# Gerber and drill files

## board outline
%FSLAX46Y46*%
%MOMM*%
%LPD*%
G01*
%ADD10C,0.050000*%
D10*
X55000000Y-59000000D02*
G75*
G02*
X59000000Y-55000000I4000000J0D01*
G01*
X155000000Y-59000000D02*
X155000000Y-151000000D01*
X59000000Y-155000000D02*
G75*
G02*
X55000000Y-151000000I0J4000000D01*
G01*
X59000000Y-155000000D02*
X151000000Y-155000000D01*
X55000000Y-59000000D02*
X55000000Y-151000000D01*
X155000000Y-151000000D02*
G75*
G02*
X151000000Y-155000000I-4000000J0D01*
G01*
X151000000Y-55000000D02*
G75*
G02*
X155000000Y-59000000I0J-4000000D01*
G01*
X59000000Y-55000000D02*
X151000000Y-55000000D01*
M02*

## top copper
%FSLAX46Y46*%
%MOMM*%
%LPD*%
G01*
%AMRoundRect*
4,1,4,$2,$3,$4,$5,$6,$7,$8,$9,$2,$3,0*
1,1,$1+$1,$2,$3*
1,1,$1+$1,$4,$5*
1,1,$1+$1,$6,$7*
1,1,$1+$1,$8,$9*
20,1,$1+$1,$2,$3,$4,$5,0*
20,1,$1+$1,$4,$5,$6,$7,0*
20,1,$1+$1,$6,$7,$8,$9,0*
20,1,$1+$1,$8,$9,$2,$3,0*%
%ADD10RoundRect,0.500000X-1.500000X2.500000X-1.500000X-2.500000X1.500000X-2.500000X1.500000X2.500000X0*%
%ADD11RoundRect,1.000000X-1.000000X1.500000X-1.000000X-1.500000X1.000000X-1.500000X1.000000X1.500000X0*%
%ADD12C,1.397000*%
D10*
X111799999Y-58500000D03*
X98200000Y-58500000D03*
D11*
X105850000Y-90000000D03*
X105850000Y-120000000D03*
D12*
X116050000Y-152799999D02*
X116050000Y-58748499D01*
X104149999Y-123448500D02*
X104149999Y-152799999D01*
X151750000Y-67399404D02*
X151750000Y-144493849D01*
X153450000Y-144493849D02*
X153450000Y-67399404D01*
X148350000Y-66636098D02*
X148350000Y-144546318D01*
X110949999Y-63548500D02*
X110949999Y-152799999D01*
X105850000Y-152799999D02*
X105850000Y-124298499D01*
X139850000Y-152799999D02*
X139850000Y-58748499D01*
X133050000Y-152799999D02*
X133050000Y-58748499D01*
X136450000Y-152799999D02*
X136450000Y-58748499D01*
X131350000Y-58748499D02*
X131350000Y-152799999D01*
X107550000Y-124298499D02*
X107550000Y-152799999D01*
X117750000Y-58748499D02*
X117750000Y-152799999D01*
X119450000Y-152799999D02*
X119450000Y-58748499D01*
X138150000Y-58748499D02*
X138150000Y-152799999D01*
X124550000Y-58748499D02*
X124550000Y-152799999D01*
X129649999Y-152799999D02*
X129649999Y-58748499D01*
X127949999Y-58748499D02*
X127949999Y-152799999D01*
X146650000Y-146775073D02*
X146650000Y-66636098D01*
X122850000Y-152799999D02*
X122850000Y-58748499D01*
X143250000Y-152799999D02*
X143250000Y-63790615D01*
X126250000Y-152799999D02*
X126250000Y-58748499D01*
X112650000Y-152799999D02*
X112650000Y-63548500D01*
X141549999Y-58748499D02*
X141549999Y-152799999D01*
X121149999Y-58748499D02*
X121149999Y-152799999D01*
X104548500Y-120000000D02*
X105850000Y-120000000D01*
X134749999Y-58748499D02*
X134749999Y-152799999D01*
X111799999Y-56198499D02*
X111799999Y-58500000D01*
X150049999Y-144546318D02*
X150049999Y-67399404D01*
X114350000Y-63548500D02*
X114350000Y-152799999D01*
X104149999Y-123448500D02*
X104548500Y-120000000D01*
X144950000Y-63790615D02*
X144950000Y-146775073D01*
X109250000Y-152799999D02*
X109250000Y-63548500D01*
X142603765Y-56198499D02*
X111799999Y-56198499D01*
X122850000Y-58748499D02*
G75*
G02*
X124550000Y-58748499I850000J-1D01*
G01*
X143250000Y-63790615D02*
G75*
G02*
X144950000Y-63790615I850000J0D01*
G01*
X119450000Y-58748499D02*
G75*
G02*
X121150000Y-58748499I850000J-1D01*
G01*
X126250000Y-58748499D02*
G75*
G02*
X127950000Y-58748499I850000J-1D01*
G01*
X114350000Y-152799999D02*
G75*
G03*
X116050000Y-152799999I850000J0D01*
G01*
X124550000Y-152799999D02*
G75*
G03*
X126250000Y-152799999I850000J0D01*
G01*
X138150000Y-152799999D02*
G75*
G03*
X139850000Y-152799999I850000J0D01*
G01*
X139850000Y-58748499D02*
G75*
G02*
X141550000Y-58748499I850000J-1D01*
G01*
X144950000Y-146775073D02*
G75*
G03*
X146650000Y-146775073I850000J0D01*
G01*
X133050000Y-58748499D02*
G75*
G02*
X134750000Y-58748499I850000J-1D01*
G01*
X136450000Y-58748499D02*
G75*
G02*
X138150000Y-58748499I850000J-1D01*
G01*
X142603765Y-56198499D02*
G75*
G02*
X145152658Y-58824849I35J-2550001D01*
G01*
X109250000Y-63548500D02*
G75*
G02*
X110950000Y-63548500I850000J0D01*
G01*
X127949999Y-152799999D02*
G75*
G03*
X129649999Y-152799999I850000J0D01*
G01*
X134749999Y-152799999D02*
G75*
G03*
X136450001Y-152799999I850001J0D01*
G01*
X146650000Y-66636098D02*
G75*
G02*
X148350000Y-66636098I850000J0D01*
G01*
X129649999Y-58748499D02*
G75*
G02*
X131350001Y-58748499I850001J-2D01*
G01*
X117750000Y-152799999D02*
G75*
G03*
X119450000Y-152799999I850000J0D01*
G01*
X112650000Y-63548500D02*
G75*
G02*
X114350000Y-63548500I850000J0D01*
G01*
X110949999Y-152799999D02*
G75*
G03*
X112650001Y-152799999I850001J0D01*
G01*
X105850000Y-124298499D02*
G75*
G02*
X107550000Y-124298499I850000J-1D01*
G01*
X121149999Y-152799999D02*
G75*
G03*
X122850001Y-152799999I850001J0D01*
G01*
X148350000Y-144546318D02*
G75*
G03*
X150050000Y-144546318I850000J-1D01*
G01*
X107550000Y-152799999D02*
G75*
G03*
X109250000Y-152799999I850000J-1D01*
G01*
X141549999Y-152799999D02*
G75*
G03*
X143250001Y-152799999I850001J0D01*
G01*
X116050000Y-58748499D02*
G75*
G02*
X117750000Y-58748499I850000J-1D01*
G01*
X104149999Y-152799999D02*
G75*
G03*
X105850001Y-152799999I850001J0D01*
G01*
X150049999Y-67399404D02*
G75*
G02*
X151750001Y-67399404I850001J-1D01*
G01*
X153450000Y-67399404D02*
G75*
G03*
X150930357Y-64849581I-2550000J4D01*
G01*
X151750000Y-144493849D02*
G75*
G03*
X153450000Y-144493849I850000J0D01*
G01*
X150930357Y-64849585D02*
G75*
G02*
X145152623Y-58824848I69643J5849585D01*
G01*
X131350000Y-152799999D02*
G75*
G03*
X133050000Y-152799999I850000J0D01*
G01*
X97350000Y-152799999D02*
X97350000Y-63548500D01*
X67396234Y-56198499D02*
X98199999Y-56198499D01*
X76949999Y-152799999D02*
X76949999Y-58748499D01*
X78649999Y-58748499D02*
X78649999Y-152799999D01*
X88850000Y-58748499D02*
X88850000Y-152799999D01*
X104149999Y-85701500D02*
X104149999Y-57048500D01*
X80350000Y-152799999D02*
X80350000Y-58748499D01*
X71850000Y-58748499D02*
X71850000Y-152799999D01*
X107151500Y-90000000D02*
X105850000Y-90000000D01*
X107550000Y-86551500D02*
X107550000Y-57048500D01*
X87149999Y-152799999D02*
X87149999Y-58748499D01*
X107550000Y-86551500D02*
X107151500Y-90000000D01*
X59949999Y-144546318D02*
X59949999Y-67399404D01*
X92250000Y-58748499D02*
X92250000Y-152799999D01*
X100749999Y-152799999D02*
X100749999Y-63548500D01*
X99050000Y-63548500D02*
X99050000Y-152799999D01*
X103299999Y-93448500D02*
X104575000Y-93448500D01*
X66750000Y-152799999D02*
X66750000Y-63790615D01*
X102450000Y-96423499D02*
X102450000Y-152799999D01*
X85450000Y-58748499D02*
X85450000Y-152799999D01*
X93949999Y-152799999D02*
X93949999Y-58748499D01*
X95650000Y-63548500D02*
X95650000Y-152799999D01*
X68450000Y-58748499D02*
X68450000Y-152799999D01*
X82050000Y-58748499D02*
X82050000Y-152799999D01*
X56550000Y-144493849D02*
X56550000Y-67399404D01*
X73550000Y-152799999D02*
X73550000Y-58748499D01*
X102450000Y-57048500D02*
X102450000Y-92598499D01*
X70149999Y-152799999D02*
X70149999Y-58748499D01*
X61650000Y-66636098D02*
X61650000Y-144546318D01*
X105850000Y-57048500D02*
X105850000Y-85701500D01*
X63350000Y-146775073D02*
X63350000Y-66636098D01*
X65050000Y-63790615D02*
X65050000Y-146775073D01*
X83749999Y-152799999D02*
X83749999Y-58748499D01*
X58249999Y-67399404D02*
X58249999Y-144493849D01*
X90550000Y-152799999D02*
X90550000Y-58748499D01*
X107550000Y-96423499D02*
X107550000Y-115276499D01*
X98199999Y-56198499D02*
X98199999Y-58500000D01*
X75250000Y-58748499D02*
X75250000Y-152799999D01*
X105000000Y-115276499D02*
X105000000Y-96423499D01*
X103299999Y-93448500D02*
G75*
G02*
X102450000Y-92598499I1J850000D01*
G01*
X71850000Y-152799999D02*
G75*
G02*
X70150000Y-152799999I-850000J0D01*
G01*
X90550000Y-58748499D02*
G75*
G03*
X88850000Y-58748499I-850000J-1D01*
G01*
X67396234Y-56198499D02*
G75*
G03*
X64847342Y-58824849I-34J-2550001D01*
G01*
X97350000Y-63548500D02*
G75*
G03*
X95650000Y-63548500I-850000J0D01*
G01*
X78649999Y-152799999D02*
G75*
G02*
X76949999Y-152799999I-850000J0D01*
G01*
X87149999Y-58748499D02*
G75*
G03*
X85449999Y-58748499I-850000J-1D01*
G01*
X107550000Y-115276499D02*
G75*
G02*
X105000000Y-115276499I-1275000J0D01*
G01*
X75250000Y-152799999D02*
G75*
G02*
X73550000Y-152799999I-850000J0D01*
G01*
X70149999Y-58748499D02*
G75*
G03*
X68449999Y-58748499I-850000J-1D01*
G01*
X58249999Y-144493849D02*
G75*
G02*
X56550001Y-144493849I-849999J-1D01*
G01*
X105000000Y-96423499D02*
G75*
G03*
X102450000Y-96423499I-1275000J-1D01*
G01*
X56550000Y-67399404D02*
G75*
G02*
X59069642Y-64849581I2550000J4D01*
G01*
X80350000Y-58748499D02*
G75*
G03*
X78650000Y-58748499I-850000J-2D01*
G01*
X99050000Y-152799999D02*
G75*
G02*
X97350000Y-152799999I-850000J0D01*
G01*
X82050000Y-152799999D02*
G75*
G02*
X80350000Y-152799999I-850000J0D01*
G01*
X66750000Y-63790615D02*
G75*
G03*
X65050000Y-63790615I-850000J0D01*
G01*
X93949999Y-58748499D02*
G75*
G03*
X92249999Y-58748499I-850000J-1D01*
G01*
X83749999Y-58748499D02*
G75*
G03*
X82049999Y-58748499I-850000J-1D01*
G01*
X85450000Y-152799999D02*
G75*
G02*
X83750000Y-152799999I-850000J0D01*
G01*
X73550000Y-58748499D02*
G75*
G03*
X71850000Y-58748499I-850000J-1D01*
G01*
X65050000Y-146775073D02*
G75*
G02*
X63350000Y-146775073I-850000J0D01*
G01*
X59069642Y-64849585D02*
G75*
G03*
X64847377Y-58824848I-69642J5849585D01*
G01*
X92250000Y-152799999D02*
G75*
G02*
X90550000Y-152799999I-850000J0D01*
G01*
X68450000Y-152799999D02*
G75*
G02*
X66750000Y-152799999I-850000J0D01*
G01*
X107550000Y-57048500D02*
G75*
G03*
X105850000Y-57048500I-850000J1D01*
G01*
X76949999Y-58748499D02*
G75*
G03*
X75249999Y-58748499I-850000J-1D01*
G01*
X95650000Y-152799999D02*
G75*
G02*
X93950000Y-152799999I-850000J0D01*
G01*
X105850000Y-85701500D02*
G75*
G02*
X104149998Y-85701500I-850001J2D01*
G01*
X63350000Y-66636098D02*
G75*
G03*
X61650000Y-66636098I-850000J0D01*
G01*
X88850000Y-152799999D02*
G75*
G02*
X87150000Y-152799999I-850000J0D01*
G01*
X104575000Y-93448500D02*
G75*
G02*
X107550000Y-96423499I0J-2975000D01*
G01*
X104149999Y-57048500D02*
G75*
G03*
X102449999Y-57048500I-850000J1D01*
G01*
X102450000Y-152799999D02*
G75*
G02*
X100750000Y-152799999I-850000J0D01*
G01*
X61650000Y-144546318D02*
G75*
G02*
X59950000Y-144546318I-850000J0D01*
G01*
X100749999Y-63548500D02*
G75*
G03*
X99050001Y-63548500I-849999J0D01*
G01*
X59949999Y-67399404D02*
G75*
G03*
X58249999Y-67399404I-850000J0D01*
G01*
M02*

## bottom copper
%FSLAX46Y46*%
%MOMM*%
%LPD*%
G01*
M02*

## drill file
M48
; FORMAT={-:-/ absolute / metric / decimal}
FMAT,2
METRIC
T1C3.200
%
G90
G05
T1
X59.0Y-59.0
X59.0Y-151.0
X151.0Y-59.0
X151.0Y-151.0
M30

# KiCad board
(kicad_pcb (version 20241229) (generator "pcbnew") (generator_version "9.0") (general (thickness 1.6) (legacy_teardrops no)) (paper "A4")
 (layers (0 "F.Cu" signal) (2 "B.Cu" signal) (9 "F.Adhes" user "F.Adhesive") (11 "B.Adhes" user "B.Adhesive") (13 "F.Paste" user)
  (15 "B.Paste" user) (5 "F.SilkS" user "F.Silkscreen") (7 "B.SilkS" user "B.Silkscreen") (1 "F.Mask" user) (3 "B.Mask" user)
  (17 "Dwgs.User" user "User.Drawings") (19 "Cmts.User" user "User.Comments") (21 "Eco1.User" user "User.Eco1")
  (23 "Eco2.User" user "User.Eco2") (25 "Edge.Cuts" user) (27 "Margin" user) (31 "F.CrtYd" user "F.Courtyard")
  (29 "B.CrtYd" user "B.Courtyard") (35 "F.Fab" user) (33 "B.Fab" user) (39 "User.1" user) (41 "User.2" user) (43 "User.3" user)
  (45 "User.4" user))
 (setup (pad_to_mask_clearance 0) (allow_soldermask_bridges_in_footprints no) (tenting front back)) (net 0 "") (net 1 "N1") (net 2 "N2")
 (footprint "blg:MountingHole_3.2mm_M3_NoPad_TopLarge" (layer "F.Cu") (at 151 59)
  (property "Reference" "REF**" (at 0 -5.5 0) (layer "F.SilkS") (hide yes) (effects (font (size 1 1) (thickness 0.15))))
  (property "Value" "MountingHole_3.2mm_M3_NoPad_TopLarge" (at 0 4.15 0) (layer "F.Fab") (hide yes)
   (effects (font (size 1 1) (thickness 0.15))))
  (pad "" np_thru_hole circle (at 0 0) (size 7.6 7.6) (drill 3.2) (layers) (zone_connect 2)))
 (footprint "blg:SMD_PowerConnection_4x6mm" (layer "F.Cu") (at 111.799999 58.5 -90)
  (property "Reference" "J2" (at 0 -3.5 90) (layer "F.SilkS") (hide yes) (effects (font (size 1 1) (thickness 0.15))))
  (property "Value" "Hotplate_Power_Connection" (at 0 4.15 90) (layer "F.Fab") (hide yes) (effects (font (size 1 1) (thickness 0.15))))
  (pad "1" smd roundrect (at 0 0 270) (size 6 4) (layers "F.Cu" "F.Mask" "F.Paste") (roundrect_rratio 0.125) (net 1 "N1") (zone_connect 2)))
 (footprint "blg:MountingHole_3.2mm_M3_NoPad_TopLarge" (layer "F.Cu") (at 59 151)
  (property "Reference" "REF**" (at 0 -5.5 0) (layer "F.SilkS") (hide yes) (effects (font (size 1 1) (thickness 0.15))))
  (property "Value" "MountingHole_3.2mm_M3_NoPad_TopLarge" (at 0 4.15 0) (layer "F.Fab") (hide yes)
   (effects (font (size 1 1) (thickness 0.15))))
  (pad "" np_thru_hole circle (at 0 0) (size 7.6 7.6) (drill 3.2) (layers) (zone_connect 2)))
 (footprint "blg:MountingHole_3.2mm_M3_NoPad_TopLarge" (layer "F.Cu") (at 151 151)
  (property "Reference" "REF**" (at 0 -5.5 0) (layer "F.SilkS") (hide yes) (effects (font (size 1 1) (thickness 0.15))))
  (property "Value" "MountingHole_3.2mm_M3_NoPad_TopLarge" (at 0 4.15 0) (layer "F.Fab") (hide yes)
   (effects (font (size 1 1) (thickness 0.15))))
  (pad "" np_thru_hole circle (at 0 0) (size 7.6 7.6) (drill 3.2) (layers) (zone_connect 2)))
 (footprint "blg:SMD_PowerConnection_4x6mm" (layer "F.Cu") (at 98.2 58.5 -90)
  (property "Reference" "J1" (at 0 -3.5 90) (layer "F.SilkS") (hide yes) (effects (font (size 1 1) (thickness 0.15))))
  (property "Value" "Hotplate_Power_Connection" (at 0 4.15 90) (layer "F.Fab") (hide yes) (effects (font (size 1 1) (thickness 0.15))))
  (pad "1" smd roundrect (at 0 0 270) (size 6 4) (layers "F.Cu" "F.Mask" "F.Paste") (roundrect_rratio 0.125) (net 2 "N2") (zone_connect 2)))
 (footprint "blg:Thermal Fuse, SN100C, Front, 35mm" (layer "F.Cu") (at 105.85 105 -90)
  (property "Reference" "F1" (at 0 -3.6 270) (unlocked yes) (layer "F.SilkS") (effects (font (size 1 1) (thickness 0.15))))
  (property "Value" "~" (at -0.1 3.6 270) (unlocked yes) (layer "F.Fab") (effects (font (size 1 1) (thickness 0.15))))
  (pad "1" smd roundrect (at -15 0 270) (size 5 4) (layers "F.Cu" "F.Mask") (roundrect_rratio 0.25) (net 2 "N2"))
  (pad "2" smd roundrect (at 15 0 270) (size 5 4) (layers "F.Cu" "F.Mask") (roundrect_rratio 0.25) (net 1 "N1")))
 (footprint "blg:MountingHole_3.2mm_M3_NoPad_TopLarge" (layer "F.Cu") (at 59 59)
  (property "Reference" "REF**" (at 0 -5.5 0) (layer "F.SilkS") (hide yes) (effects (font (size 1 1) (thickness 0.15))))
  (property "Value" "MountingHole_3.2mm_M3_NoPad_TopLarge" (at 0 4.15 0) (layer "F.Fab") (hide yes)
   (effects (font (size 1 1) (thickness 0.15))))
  (pad "" np_thru_hole circle (at 0 0) (size 7.6 7.6) (drill 3.2) (layers) (zone_connect 2)))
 (gr_arc (start 55 59) (mid 56.171573 56.171573) (end 59 55) (stroke (width 0.05) (type solid)) (layer "Edge.Cuts"))
 (gr_line (start 155 59) (end 155 151) (stroke (width 0.05) (type default)) (layer "Edge.Cuts"))
 (gr_arc (start 59 155) (mid 56.171573 153.828427) (end 55 151) (stroke (width 0.05) (type solid)) (layer "Edge.Cuts"))
 (gr_line (start 59 155) (end 151 155) (stroke (width 0.05) (type default)) (layer "Edge.Cuts"))
 (gr_line (start 55 59) (end 55 151) (stroke (width 0.05) (type default)) (layer "Edge.Cuts"))
 (gr_arc (start 155 151) (mid 153.828427 153.828427) (end 151 155) (stroke (width 0.05) (type solid)) (layer "Edge.Cuts"))
 (gr_arc (start 151 55) (mid 153.828427 56.171573) (end 155 59) (stroke (width 0.05) (type solid)) (layer "Edge.Cuts"))
 (gr_line (start 59 55) (end 151 55) (stroke (width 0.05) (type default)) (layer "Edge.Cuts"))
 (segment (start 116.05 152.799999) (end 116.05 58.748499) (width 1.397) (layer "F.Cu") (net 1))
 (segment (start 104.149999 123.4485) (end 104.149999 152.799999) (width 1.397) (layer "F.Cu") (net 1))
 (segment (start 151.75 67.399404) (end 151.75 144.493849) (width 1.397) (layer "F.Cu") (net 1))
 (segment (start 153.45 144.493849) (end 153.45 67.399404) (width 1.397) (layer "F.Cu") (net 1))
 (segment (start 148.35 66.636098) (end 148.35 144.546318) (width 1.397) (layer "F.Cu") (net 1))
 (segment (start 110.949999 63.5485) (end 110.949999 152.799999) (width 1.397) (layer "F.Cu") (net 1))
 (segment (start 105.85 152.799999) (end 105.85 124.298499) (width 1.397) (layer "F.Cu") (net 1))
 (segment (start 139.85 152.799999) (end 139.85 58.748499) (width 1.397) (layer "F.Cu") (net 1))
 (segment (start 133.05 152.799999) (end 133.05 58.748499) (width 1.397) (layer "F.Cu") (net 1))
 (segment (start 136.45 152.799999) (end 136.45 58.748499) (width 1.397) (layer "F.Cu") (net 1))
 (segment (start 131.35 58.748499) (end 131.35 152.799999) (width 1.397) (layer "F.Cu") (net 1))
 (segment (start 107.55 124.298499) (end 107.55 152.799999) (width 1.397) (layer "F.Cu") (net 1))
 (segment (start 117.75 58.748499) (end 117.75 152.799999) (width 1.397) (layer "F.Cu") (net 1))
 (segment (start 119.45 152.799999) (end 119.45 58.748499) (width 1.397) (layer "F.Cu") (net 1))
 (segment (start 138.15 58.748499) (end 138.15 152.799999) (width 1.397) (layer "F.Cu") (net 1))
 (segment (start 124.55 58.748499) (end 124.55 152.799999) (width 1.397) (layer "F.Cu") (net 1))
 (segment (start 129.649999 152.799999) (end 129.649999 58.748499) (width 1.397) (layer "F.Cu") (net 1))
 (segment (start 127.949999 58.748499) (end 127.949999 152.799999) (width 1.397) (layer "F.Cu") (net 1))
 (segment (start 146.65 146.775073) (end 146.65 66.636098) (width 1.397) (layer "F.Cu") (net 1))
 (segment (start 122.85 152.799999) (end 122.85 58.748499) (width 1.397) (layer "F.Cu") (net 1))
 (segment (start 143.25 152.799999) (end 143.25 63.790615) (width 1.397) (layer "F.Cu") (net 1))
 (segment (start 126.25 152.799999) (end 126.25 58.748499) (width 1.397) (layer "F.Cu") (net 1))
 (segment (start 112.65 152.799999) (end 112.65 63.5485) (width 1.397) (layer "F.Cu") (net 1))
 (segment (start 141.549999 58.748499) (end 141.549999 152.799999) (width 1.397) (layer "F.Cu") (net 1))
 (segment (start 121.149999 58.748499) (end 121.149999 152.799999) (width 1.397) (layer "F.Cu") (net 1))
 (segment (start 104.5485 120) (end 105.85 120) (width 1.397) (layer "F.Cu") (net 1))
 (segment (start 134.749999 58.748499) (end 134.749999 152.799999) (width 1.397) (layer "F.Cu") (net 1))
 (segment (start 111.799999 56.198499) (end 111.799999 58.5) (width 1.397) (layer "F.Cu") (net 1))
 (segment (start 150.049999 144.546318) (end 150.049999 67.399404) (width 1.397) (layer "F.Cu") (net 1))
 (segment (start 114.35 63.5485) (end 114.35 152.799999) (width 1.397) (layer "F.Cu") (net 1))
 (segment (start 104.149999 123.4485) (end 104.5485 120) (width 1.397) (layer "F.Cu") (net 1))
 (segment (start 144.95 63.790615) (end 144.95 146.775073) (width 1.397) (layer "F.Cu") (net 1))
 (segment (start 109.25 152.799999) (end 109.25 63.5485) (width 1.397) (layer "F.Cu") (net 1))
 (segment (start 142.603765 56.198499) (end 111.799999 56.198499) (width 1.397) (layer "F.Cu") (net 1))
 (arc (start 122.85 58.748499) (mid 123.699999 57.8985) (end 124.55 58.748499) (width 1.397) (layer "F.Cu") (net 1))
 (arc (start 143.25 63.790615) (mid 144.1 62.940615) (end 144.95 63.790615) (width 1.397) (layer "F.Cu") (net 1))
 (arc (start 119.45 58.748499) (mid 120.3 57.8985) (end 121.149999 58.748499) (width 1.397) (layer "F.Cu") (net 1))
 (arc (start 126.25 58.748499) (mid 127.1 57.8985) (end 127.949999 58.748499) (width 1.397) (layer "F.Cu") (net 1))
 (arc (start 114.35 152.799999) (mid 115.2 153.649999) (end 116.05 152.799999) (width 1.397) (layer "F.Cu") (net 1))
 (arc (start 124.55 152.799999) (mid 125.399999 153.649999) (end 126.25 152.799999) (width 1.397) (layer "F.Cu") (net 1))
 (arc (start 138.15 152.799999) (mid 138.999999 153.649999) (end 139.85 152.799999) (width 1.397) (layer "F.Cu") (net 1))
 (arc (start 139.85 58.748499) (mid 140.7 57.8985) (end 141.549999 58.748499) (width 1.397) (layer "F.Cu") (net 1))
 (arc (start 144.95 146.775073) (mid 145.799999 147.625073) (end 146.65 146.775073) (width 1.397) (layer "F.Cu") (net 1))
 (arc (start 133.05 58.748499) (mid 133.899999 57.8985) (end 134.749999 58.748499) (width 1.397) (layer "F.Cu") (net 1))
 (arc (start 136.45 58.748499) (mid 137.3 57.8985) (end 138.15 58.748499) (width 1.397) (layer "F.Cu") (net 1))
 (arc (start 142.603765 56.198499) (mid 144.433682 56.972576) (end 145.152622 58.824848) (width 1.397) (layer "F.Cu") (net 1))
 (arc (start 109.25 63.5485) (mid 110.1 62.6985) (end 110.949999 63.5485) (width 1.397) (layer "F.Cu") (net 1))
 (arc (start 127.949999 152.799999) (mid 128.8 153.649999) (end 129.649999 152.799999) (width 1.397) (layer "F.Cu") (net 1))
 (arc (start 134.749999 152.799999) (mid 135.6 153.649999) (end 136.45 152.799999) (width 1.397) (layer "F.Cu") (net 1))
 (arc (start 146.65 66.636098) (mid 147.5 65.786098) (end 148.35 66.636098) (width 1.397) (layer "F.Cu") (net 1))
 (arc (start 129.649999 58.748499) (mid 130.5 57.8985) (end 131.35 58.748499) (width 1.397) (layer "F.Cu") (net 1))
 (arc (start 117.75 152.799999) (mid 118.6 153.649999) (end 119.45 152.799999) (width 1.397) (layer "F.Cu") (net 1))
 (arc (start 112.65 63.5485) (mid 113.499999 62.6985) (end 114.35 63.5485) (width 1.397) (layer "F.Cu") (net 1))
 (arc (start 110.949999 152.799999) (mid 111.8 153.649999) (end 112.65 152.799999) (width 1.397) (layer "F.Cu") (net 1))
 (arc (start 105.85 124.298499) (mid 106.699999 123.4485) (end 107.55 124.298499) (width 1.397) (layer "F.Cu") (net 1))
 (arc (start 121.149999 152.799999) (mid 122 153.649999) (end 122.85 152.799999) (width 1.397) (layer "F.Cu") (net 1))
 (arc (start 148.35 144.546318) (mid 149.2 145.396318) (end 150.049999 144.546318) (width 1.397) (layer "F.Cu") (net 1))
 (arc (start 107.55 152.799999) (mid 108.399999 153.649999) (end 109.249999 152.799999) (width 1.397) (layer "F.Cu") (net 1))
 (arc (start 141.549999 152.799999) (mid 142.4 153.649999) (end 143.25 152.799999) (width 1.397) (layer "F.Cu") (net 1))
 (arc (start 116.05 58.748499) (mid 116.899999 57.8985) (end 117.75 58.748499) (width 1.397) (layer "F.Cu") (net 1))
 (arc (start 104.149999 152.799999) (mid 105 153.649999) (end 105.85 152.799999) (width 1.397) (layer "F.Cu") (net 1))
 (arc (start 150.049999 67.399404) (mid 150.9 66.549404) (end 151.75 67.399404) (width 1.397) (layer "F.Cu") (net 1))
 (arc (start 153.45 67.399404) (mid 152.737249 65.631068) (end 150.930357 64.849585) (width 1.397) (layer "F.Cu") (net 1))
 (arc (start 151.75 144.493849) (mid 152.6 145.343849) (end 153.45 144.493849) (width 1.397) (layer "F.Cu") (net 1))
 (arc (start 150.930357 64.849585) (mid 146.777779 63.049117) (end 145.152622 58.824848) (width 1.397) (layer "F.Cu") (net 1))
 (arc (start 131.35 152.799999) (mid 132.199999 153.649999) (end 133.05 152.799999) (width 1.397) (layer "F.Cu") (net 1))
 (segment (start 97.35 152.799999) (end 97.35 63.5485) (width 1.397) (layer "F.Cu") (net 2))
 (segment (start 67.396234 56.198499) (end 98.199999 56.198499) (width 1.397) (layer "F.Cu") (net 2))
 (segment (start 76.949999 152.799999) (end 76.949999 58.748499) (width 1.397) (layer "F.Cu") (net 2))
 (segment (start 78.649999 58.748499) (end 78.649999 152.799999) (width 1.397) (layer "F.Cu") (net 2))
 (segment (start 88.85 58.748499) (end 88.85 152.799999) (width 1.397) (layer "F.Cu") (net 2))
 (segment (start 104.149999 85.7015) (end 104.149999 57.0485) (width 1.397) (layer "F.Cu") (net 2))
 (segment (start 80.35 152.799999) (end 80.35 58.748499) (width 1.397) (layer "F.Cu") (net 2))
 (segment (start 71.85 58.748499) (end 71.85 152.799999) (width 1.397) (layer "F.Cu") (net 2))
 (segment (start 107.1515 90) (end 105.85 90) (width 1.397) (layer "F.Cu") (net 2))
 (segment (start 107.55 86.5515) (end 107.55 57.0485) (width 1.397) (layer "F.Cu") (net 2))
 (segment (start 87.149999 152.799999) (end 87.149999 58.748499) (width 1.397) (layer "F.Cu") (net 2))
 (segment (start 107.55 86.5515) (end 107.1515 90) (width 1.397) (layer "F.Cu") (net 2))
 (segment (start 59.949999 144.546318) (end 59.949999 67.399404) (width 1.397) (layer "F.Cu") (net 2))
 (segment (start 92.25 58.748499) (end 92.25 152.799999) (width 1.397) (layer "F.Cu") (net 2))
 (segment (start 100.749999 152.799999) (end 100.749999 63.5485) (width 1.397) (layer "F.Cu") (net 2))
 (segment (start 99.05 63.5485) (end 99.05 152.799999) (width 1.397) (layer "F.Cu") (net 2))
 (segment (start 103.299999 93.4485) (end 104.575 93.4485) (width 1.397) (layer "F.Cu") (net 2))
 (segment (start 66.75 152.799999) (end 66.75 63.790615) (width 1.397) (layer "F.Cu") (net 2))
 (segment (start 102.45 96.423499) (end 102.45 152.799999) (width 1.397) (layer "F.Cu") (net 2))
 (segment (start 85.45 58.748499) (end 85.45 152.799999) (width 1.397) (layer "F.Cu") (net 2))
 (segment (start 93.949999 152.799999) (end 93.949999 58.748499) (width 1.397) (layer "F.Cu") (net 2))
 (segment (start 95.65 63.5485) (end 95.65 152.799999) (width 1.397) (layer "F.Cu") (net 2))
 (segment (start 68.45 58.748499) (end 68.45 152.799999) (width 1.397) (layer "F.Cu") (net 2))
 (segment (start 82.05 58.748499) (end 82.05 152.799999) (width 1.397) (layer "F.Cu") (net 2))
 (segment (start 56.55 144.493849) (end 56.55 67.399404) (width 1.397) (layer "F.Cu") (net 2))
 (segment (start 73.55 152.799999) (end 73.55 58.748499) (width 1.397) (layer "F.Cu") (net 2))
 (segment (start 102.45 57.0485) (end 102.45 92.598499) (width 1.397) (layer "F.Cu") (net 2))
 (segment (start 70.149999 152.799999) (end 70.149999 58.748499) (width 1.397) (layer "F.Cu") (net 2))
 (segment (start 61.65 66.636098) (end 61.65 144.546318) (width 1.397) (layer "F.Cu") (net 2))
 (segment (start 105.85 57.0485) (end 105.85 85.7015) (width 1.397) (layer "F.Cu") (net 2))
 (segment (start 63.35 146.775073) (end 63.35 66.636098) (width 1.397) (layer "F.Cu") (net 2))
 (segment (start 65.05 63.790615) (end 65.05 146.775073) (width 1.397) (layer "F.Cu") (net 2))
 (segment (start 83.749999 152.799999) (end 83.749999 58.748499) (width 1.397) (layer "F.Cu") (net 2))
 (segment (start 58.249999 67.399404) (end 58.249999 144.493849) (width 1.397) (layer "F.Cu") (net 2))
 (segment (start 90.55 152.799999) (end 90.55 58.748499) (width 1.397) (layer "F.Cu") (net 2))
 (segment (start 107.55 96.423499) (end 107.55 115.276499) (width 1.397) (layer "F.Cu") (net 2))
 (segment (start 98.199999 56.198499) (end 98.199999 58.5) (width 1.397) (layer "F.Cu") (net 2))
 (segment (start 75.25 58.748499) (end 75.25 152.799999) (width 1.397) (layer "F.Cu") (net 2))
 (segment (start 105 115.276499) (end 105 96.423499) (width 1.397) (layer "F.Cu") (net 2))
 (arc (start 103.299999 93.4485) (mid 102.698959 93.19954) (end 102.45 92.598499) (width 1.397) (layer "F.Cu") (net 2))
 (arc (start 71.85 152.799999) (mid 71 153.649999) (end 70.149999 152.799999) (width 1.397) (layer "F.Cu") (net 2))
 (arc (start 90.55 58.748499) (mid 89.7 57.8985) (end 88.85 58.748499) (width 1.397) (layer "F.Cu") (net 2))
 (arc (start 67.396234 56.198499) (mid 65.566317 56.972576) (end 64.847377 58.824848) (width 1.397) (layer "F.Cu") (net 2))
 (arc (start 97.35 63.5485) (mid 96.5 62.6985) (end 95.65 63.5485) (width 1.397) (layer "F.Cu") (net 2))
 (arc (start 78.649999 152.799999) (mid 77.8 153.649999) (end 76.949999 152.799999) (width 1.397) (layer "F.Cu") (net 2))
 (arc (start 87.149999 58.748499) (mid 86.3 57.8985) (end 85.45 58.748499) (width 1.397) (layer "F.Cu") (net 2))
 (arc (start 107.55 115.276499) (mid 106.274999 116.551499) (end 105 115.276499) (width 1.397) (layer "F.Cu") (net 2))
 (arc (start 75.25 152.799999) (mid 74.399999 153.649999) (end 73.55 152.799999) (width 1.397) (layer "F.Cu") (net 2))
 (arc (start 70.149999 58.748499) (mid 69.3 57.8985) (end 68.45 58.748499) (width 1.397) (layer "F.Cu") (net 2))
 (arc (start 58.249999 144.493849) (mid 57.4 145.343849) (end 56.55 144.493849) (width 1.397) (layer "F.Cu") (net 2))
 (arc (start 105 96.423499) (mid 103.725 95.1485) (end 102.45 96.423499) (width 1.397) (layer "F.Cu") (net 2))
 (arc (start 56.55 67.399404) (mid 57.26275 65.631068) (end 59.069642 64.849585) (width 1.397) (layer "F.Cu") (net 2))
 (arc (start 80.35 58.748499) (mid 79.5 57.8985) (end 78.649999 58.748499) (width 1.397) (layer "F.Cu") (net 2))
 (arc (start 99.05 152.799999) (mid 98.199999 153.649999) (end 97.35 152.799999) (width 1.397) (layer "F.Cu") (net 2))
 (arc (start 82.05 152.799999) (mid 81.199999 153.649999) (end 80.35 152.799999) (width 1.397) (layer "F.Cu") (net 2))
 (arc (start 66.75 63.790615) (mid 65.9 62.940615) (end 65.05 63.790615) (width 1.397) (layer "F.Cu") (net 2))
 (arc (start 93.949999 58.748499) (mid 93.1 57.8985) (end 92.25 58.748499) (width 1.397) (layer "F.Cu") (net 2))
 (arc (start 83.749999 58.748499) (mid 82.9 57.8985) (end 82.05 58.748499) (width 1.397) (layer "F.Cu") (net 2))
 (arc (start 85.45 152.799999) (mid 84.6 153.649999) (end 83.749999 152.799999) (width 1.397) (layer "F.Cu") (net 2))
 (arc (start 73.55 58.748499) (mid 72.7 57.8985) (end 71.85 58.748499) (width 1.397) (layer "F.Cu") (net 2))
 (arc (start 65.05 146.775073) (mid 64.199999 147.625073) (end 63.35 146.775073) (width 1.397) (layer "F.Cu") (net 2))
 (arc (start 59.069642 64.849585) (mid 63.22222 63.049117) (end 64.847377 58.824848) (width 1.397) (layer "F.Cu") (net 2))
 (arc (start 92.25 152.799999) (mid 91.399999 153.649999) (end 90.55 152.799999) (width 1.397) (layer "F.Cu") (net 2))
 (arc (start 68.45 152.799999) (mid 67.6 153.649999) (end 66.75 152.799999) (width 1.397) (layer "F.Cu") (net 2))
 (arc (start 107.55 57.0485) (mid 106.699999 56.198499) (end 105.85 57.0485) (width 1.397) (layer "F.Cu") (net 2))
 (arc (start 76.949999 58.748499) (mid 76.1 57.8985) (end 75.25 58.748499) (width 1.397) (layer "F.Cu") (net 2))
 (arc (start 95.65 152.799999) (mid 94.8 153.649999) (end 93.949999 152.799999) (width 1.397) (layer "F.Cu") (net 2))
 (arc (start 105.85 85.7015) (mid 105 86.551499) (end 104.149999 85.7015) (width 1.397) (layer "F.Cu") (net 2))
 (arc (start 63.35 66.636098) (mid 62.5 65.786098) (end 61.65 66.636098) (width 1.397) (layer "F.Cu") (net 2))
 (arc (start 88.85 152.799999) (mid 88 153.649999) (end 87.149999 152.799999) (width 1.397) (layer "F.Cu") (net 2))
 (arc (start 104.575 93.4485) (mid 106.678642 94.319857) (end 107.55 96.423499) (width 1.397) (layer "F.Cu") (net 2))
 (arc (start 104.149999 57.0485) (mid 103.299999 56.198499) (end 102.45 57.0485) (width 1.397) (layer "F.Cu") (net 2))
 (arc (start 102.45 152.799999) (mid 101.6 153.649999) (end 100.749999 152.799999) (width 1.397) (layer "F.Cu") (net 2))
 (arc (start 61.65 144.546318) (mid 60.8 145.396318) (end 59.949999 144.546318) (width 1.397) (layer "F.Cu") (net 2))
 (arc (start 100.749999 63.5485) (mid 99.899999 62.6985) (end 99.05 63.5485) (width 1.397) (layer "F.Cu") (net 2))
 (arc (start 59.949999 67.399404) (mid 59.1 66.549404) (end 58.249999 67.399404) (width 1.397) (layer "F.Cu") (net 2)))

